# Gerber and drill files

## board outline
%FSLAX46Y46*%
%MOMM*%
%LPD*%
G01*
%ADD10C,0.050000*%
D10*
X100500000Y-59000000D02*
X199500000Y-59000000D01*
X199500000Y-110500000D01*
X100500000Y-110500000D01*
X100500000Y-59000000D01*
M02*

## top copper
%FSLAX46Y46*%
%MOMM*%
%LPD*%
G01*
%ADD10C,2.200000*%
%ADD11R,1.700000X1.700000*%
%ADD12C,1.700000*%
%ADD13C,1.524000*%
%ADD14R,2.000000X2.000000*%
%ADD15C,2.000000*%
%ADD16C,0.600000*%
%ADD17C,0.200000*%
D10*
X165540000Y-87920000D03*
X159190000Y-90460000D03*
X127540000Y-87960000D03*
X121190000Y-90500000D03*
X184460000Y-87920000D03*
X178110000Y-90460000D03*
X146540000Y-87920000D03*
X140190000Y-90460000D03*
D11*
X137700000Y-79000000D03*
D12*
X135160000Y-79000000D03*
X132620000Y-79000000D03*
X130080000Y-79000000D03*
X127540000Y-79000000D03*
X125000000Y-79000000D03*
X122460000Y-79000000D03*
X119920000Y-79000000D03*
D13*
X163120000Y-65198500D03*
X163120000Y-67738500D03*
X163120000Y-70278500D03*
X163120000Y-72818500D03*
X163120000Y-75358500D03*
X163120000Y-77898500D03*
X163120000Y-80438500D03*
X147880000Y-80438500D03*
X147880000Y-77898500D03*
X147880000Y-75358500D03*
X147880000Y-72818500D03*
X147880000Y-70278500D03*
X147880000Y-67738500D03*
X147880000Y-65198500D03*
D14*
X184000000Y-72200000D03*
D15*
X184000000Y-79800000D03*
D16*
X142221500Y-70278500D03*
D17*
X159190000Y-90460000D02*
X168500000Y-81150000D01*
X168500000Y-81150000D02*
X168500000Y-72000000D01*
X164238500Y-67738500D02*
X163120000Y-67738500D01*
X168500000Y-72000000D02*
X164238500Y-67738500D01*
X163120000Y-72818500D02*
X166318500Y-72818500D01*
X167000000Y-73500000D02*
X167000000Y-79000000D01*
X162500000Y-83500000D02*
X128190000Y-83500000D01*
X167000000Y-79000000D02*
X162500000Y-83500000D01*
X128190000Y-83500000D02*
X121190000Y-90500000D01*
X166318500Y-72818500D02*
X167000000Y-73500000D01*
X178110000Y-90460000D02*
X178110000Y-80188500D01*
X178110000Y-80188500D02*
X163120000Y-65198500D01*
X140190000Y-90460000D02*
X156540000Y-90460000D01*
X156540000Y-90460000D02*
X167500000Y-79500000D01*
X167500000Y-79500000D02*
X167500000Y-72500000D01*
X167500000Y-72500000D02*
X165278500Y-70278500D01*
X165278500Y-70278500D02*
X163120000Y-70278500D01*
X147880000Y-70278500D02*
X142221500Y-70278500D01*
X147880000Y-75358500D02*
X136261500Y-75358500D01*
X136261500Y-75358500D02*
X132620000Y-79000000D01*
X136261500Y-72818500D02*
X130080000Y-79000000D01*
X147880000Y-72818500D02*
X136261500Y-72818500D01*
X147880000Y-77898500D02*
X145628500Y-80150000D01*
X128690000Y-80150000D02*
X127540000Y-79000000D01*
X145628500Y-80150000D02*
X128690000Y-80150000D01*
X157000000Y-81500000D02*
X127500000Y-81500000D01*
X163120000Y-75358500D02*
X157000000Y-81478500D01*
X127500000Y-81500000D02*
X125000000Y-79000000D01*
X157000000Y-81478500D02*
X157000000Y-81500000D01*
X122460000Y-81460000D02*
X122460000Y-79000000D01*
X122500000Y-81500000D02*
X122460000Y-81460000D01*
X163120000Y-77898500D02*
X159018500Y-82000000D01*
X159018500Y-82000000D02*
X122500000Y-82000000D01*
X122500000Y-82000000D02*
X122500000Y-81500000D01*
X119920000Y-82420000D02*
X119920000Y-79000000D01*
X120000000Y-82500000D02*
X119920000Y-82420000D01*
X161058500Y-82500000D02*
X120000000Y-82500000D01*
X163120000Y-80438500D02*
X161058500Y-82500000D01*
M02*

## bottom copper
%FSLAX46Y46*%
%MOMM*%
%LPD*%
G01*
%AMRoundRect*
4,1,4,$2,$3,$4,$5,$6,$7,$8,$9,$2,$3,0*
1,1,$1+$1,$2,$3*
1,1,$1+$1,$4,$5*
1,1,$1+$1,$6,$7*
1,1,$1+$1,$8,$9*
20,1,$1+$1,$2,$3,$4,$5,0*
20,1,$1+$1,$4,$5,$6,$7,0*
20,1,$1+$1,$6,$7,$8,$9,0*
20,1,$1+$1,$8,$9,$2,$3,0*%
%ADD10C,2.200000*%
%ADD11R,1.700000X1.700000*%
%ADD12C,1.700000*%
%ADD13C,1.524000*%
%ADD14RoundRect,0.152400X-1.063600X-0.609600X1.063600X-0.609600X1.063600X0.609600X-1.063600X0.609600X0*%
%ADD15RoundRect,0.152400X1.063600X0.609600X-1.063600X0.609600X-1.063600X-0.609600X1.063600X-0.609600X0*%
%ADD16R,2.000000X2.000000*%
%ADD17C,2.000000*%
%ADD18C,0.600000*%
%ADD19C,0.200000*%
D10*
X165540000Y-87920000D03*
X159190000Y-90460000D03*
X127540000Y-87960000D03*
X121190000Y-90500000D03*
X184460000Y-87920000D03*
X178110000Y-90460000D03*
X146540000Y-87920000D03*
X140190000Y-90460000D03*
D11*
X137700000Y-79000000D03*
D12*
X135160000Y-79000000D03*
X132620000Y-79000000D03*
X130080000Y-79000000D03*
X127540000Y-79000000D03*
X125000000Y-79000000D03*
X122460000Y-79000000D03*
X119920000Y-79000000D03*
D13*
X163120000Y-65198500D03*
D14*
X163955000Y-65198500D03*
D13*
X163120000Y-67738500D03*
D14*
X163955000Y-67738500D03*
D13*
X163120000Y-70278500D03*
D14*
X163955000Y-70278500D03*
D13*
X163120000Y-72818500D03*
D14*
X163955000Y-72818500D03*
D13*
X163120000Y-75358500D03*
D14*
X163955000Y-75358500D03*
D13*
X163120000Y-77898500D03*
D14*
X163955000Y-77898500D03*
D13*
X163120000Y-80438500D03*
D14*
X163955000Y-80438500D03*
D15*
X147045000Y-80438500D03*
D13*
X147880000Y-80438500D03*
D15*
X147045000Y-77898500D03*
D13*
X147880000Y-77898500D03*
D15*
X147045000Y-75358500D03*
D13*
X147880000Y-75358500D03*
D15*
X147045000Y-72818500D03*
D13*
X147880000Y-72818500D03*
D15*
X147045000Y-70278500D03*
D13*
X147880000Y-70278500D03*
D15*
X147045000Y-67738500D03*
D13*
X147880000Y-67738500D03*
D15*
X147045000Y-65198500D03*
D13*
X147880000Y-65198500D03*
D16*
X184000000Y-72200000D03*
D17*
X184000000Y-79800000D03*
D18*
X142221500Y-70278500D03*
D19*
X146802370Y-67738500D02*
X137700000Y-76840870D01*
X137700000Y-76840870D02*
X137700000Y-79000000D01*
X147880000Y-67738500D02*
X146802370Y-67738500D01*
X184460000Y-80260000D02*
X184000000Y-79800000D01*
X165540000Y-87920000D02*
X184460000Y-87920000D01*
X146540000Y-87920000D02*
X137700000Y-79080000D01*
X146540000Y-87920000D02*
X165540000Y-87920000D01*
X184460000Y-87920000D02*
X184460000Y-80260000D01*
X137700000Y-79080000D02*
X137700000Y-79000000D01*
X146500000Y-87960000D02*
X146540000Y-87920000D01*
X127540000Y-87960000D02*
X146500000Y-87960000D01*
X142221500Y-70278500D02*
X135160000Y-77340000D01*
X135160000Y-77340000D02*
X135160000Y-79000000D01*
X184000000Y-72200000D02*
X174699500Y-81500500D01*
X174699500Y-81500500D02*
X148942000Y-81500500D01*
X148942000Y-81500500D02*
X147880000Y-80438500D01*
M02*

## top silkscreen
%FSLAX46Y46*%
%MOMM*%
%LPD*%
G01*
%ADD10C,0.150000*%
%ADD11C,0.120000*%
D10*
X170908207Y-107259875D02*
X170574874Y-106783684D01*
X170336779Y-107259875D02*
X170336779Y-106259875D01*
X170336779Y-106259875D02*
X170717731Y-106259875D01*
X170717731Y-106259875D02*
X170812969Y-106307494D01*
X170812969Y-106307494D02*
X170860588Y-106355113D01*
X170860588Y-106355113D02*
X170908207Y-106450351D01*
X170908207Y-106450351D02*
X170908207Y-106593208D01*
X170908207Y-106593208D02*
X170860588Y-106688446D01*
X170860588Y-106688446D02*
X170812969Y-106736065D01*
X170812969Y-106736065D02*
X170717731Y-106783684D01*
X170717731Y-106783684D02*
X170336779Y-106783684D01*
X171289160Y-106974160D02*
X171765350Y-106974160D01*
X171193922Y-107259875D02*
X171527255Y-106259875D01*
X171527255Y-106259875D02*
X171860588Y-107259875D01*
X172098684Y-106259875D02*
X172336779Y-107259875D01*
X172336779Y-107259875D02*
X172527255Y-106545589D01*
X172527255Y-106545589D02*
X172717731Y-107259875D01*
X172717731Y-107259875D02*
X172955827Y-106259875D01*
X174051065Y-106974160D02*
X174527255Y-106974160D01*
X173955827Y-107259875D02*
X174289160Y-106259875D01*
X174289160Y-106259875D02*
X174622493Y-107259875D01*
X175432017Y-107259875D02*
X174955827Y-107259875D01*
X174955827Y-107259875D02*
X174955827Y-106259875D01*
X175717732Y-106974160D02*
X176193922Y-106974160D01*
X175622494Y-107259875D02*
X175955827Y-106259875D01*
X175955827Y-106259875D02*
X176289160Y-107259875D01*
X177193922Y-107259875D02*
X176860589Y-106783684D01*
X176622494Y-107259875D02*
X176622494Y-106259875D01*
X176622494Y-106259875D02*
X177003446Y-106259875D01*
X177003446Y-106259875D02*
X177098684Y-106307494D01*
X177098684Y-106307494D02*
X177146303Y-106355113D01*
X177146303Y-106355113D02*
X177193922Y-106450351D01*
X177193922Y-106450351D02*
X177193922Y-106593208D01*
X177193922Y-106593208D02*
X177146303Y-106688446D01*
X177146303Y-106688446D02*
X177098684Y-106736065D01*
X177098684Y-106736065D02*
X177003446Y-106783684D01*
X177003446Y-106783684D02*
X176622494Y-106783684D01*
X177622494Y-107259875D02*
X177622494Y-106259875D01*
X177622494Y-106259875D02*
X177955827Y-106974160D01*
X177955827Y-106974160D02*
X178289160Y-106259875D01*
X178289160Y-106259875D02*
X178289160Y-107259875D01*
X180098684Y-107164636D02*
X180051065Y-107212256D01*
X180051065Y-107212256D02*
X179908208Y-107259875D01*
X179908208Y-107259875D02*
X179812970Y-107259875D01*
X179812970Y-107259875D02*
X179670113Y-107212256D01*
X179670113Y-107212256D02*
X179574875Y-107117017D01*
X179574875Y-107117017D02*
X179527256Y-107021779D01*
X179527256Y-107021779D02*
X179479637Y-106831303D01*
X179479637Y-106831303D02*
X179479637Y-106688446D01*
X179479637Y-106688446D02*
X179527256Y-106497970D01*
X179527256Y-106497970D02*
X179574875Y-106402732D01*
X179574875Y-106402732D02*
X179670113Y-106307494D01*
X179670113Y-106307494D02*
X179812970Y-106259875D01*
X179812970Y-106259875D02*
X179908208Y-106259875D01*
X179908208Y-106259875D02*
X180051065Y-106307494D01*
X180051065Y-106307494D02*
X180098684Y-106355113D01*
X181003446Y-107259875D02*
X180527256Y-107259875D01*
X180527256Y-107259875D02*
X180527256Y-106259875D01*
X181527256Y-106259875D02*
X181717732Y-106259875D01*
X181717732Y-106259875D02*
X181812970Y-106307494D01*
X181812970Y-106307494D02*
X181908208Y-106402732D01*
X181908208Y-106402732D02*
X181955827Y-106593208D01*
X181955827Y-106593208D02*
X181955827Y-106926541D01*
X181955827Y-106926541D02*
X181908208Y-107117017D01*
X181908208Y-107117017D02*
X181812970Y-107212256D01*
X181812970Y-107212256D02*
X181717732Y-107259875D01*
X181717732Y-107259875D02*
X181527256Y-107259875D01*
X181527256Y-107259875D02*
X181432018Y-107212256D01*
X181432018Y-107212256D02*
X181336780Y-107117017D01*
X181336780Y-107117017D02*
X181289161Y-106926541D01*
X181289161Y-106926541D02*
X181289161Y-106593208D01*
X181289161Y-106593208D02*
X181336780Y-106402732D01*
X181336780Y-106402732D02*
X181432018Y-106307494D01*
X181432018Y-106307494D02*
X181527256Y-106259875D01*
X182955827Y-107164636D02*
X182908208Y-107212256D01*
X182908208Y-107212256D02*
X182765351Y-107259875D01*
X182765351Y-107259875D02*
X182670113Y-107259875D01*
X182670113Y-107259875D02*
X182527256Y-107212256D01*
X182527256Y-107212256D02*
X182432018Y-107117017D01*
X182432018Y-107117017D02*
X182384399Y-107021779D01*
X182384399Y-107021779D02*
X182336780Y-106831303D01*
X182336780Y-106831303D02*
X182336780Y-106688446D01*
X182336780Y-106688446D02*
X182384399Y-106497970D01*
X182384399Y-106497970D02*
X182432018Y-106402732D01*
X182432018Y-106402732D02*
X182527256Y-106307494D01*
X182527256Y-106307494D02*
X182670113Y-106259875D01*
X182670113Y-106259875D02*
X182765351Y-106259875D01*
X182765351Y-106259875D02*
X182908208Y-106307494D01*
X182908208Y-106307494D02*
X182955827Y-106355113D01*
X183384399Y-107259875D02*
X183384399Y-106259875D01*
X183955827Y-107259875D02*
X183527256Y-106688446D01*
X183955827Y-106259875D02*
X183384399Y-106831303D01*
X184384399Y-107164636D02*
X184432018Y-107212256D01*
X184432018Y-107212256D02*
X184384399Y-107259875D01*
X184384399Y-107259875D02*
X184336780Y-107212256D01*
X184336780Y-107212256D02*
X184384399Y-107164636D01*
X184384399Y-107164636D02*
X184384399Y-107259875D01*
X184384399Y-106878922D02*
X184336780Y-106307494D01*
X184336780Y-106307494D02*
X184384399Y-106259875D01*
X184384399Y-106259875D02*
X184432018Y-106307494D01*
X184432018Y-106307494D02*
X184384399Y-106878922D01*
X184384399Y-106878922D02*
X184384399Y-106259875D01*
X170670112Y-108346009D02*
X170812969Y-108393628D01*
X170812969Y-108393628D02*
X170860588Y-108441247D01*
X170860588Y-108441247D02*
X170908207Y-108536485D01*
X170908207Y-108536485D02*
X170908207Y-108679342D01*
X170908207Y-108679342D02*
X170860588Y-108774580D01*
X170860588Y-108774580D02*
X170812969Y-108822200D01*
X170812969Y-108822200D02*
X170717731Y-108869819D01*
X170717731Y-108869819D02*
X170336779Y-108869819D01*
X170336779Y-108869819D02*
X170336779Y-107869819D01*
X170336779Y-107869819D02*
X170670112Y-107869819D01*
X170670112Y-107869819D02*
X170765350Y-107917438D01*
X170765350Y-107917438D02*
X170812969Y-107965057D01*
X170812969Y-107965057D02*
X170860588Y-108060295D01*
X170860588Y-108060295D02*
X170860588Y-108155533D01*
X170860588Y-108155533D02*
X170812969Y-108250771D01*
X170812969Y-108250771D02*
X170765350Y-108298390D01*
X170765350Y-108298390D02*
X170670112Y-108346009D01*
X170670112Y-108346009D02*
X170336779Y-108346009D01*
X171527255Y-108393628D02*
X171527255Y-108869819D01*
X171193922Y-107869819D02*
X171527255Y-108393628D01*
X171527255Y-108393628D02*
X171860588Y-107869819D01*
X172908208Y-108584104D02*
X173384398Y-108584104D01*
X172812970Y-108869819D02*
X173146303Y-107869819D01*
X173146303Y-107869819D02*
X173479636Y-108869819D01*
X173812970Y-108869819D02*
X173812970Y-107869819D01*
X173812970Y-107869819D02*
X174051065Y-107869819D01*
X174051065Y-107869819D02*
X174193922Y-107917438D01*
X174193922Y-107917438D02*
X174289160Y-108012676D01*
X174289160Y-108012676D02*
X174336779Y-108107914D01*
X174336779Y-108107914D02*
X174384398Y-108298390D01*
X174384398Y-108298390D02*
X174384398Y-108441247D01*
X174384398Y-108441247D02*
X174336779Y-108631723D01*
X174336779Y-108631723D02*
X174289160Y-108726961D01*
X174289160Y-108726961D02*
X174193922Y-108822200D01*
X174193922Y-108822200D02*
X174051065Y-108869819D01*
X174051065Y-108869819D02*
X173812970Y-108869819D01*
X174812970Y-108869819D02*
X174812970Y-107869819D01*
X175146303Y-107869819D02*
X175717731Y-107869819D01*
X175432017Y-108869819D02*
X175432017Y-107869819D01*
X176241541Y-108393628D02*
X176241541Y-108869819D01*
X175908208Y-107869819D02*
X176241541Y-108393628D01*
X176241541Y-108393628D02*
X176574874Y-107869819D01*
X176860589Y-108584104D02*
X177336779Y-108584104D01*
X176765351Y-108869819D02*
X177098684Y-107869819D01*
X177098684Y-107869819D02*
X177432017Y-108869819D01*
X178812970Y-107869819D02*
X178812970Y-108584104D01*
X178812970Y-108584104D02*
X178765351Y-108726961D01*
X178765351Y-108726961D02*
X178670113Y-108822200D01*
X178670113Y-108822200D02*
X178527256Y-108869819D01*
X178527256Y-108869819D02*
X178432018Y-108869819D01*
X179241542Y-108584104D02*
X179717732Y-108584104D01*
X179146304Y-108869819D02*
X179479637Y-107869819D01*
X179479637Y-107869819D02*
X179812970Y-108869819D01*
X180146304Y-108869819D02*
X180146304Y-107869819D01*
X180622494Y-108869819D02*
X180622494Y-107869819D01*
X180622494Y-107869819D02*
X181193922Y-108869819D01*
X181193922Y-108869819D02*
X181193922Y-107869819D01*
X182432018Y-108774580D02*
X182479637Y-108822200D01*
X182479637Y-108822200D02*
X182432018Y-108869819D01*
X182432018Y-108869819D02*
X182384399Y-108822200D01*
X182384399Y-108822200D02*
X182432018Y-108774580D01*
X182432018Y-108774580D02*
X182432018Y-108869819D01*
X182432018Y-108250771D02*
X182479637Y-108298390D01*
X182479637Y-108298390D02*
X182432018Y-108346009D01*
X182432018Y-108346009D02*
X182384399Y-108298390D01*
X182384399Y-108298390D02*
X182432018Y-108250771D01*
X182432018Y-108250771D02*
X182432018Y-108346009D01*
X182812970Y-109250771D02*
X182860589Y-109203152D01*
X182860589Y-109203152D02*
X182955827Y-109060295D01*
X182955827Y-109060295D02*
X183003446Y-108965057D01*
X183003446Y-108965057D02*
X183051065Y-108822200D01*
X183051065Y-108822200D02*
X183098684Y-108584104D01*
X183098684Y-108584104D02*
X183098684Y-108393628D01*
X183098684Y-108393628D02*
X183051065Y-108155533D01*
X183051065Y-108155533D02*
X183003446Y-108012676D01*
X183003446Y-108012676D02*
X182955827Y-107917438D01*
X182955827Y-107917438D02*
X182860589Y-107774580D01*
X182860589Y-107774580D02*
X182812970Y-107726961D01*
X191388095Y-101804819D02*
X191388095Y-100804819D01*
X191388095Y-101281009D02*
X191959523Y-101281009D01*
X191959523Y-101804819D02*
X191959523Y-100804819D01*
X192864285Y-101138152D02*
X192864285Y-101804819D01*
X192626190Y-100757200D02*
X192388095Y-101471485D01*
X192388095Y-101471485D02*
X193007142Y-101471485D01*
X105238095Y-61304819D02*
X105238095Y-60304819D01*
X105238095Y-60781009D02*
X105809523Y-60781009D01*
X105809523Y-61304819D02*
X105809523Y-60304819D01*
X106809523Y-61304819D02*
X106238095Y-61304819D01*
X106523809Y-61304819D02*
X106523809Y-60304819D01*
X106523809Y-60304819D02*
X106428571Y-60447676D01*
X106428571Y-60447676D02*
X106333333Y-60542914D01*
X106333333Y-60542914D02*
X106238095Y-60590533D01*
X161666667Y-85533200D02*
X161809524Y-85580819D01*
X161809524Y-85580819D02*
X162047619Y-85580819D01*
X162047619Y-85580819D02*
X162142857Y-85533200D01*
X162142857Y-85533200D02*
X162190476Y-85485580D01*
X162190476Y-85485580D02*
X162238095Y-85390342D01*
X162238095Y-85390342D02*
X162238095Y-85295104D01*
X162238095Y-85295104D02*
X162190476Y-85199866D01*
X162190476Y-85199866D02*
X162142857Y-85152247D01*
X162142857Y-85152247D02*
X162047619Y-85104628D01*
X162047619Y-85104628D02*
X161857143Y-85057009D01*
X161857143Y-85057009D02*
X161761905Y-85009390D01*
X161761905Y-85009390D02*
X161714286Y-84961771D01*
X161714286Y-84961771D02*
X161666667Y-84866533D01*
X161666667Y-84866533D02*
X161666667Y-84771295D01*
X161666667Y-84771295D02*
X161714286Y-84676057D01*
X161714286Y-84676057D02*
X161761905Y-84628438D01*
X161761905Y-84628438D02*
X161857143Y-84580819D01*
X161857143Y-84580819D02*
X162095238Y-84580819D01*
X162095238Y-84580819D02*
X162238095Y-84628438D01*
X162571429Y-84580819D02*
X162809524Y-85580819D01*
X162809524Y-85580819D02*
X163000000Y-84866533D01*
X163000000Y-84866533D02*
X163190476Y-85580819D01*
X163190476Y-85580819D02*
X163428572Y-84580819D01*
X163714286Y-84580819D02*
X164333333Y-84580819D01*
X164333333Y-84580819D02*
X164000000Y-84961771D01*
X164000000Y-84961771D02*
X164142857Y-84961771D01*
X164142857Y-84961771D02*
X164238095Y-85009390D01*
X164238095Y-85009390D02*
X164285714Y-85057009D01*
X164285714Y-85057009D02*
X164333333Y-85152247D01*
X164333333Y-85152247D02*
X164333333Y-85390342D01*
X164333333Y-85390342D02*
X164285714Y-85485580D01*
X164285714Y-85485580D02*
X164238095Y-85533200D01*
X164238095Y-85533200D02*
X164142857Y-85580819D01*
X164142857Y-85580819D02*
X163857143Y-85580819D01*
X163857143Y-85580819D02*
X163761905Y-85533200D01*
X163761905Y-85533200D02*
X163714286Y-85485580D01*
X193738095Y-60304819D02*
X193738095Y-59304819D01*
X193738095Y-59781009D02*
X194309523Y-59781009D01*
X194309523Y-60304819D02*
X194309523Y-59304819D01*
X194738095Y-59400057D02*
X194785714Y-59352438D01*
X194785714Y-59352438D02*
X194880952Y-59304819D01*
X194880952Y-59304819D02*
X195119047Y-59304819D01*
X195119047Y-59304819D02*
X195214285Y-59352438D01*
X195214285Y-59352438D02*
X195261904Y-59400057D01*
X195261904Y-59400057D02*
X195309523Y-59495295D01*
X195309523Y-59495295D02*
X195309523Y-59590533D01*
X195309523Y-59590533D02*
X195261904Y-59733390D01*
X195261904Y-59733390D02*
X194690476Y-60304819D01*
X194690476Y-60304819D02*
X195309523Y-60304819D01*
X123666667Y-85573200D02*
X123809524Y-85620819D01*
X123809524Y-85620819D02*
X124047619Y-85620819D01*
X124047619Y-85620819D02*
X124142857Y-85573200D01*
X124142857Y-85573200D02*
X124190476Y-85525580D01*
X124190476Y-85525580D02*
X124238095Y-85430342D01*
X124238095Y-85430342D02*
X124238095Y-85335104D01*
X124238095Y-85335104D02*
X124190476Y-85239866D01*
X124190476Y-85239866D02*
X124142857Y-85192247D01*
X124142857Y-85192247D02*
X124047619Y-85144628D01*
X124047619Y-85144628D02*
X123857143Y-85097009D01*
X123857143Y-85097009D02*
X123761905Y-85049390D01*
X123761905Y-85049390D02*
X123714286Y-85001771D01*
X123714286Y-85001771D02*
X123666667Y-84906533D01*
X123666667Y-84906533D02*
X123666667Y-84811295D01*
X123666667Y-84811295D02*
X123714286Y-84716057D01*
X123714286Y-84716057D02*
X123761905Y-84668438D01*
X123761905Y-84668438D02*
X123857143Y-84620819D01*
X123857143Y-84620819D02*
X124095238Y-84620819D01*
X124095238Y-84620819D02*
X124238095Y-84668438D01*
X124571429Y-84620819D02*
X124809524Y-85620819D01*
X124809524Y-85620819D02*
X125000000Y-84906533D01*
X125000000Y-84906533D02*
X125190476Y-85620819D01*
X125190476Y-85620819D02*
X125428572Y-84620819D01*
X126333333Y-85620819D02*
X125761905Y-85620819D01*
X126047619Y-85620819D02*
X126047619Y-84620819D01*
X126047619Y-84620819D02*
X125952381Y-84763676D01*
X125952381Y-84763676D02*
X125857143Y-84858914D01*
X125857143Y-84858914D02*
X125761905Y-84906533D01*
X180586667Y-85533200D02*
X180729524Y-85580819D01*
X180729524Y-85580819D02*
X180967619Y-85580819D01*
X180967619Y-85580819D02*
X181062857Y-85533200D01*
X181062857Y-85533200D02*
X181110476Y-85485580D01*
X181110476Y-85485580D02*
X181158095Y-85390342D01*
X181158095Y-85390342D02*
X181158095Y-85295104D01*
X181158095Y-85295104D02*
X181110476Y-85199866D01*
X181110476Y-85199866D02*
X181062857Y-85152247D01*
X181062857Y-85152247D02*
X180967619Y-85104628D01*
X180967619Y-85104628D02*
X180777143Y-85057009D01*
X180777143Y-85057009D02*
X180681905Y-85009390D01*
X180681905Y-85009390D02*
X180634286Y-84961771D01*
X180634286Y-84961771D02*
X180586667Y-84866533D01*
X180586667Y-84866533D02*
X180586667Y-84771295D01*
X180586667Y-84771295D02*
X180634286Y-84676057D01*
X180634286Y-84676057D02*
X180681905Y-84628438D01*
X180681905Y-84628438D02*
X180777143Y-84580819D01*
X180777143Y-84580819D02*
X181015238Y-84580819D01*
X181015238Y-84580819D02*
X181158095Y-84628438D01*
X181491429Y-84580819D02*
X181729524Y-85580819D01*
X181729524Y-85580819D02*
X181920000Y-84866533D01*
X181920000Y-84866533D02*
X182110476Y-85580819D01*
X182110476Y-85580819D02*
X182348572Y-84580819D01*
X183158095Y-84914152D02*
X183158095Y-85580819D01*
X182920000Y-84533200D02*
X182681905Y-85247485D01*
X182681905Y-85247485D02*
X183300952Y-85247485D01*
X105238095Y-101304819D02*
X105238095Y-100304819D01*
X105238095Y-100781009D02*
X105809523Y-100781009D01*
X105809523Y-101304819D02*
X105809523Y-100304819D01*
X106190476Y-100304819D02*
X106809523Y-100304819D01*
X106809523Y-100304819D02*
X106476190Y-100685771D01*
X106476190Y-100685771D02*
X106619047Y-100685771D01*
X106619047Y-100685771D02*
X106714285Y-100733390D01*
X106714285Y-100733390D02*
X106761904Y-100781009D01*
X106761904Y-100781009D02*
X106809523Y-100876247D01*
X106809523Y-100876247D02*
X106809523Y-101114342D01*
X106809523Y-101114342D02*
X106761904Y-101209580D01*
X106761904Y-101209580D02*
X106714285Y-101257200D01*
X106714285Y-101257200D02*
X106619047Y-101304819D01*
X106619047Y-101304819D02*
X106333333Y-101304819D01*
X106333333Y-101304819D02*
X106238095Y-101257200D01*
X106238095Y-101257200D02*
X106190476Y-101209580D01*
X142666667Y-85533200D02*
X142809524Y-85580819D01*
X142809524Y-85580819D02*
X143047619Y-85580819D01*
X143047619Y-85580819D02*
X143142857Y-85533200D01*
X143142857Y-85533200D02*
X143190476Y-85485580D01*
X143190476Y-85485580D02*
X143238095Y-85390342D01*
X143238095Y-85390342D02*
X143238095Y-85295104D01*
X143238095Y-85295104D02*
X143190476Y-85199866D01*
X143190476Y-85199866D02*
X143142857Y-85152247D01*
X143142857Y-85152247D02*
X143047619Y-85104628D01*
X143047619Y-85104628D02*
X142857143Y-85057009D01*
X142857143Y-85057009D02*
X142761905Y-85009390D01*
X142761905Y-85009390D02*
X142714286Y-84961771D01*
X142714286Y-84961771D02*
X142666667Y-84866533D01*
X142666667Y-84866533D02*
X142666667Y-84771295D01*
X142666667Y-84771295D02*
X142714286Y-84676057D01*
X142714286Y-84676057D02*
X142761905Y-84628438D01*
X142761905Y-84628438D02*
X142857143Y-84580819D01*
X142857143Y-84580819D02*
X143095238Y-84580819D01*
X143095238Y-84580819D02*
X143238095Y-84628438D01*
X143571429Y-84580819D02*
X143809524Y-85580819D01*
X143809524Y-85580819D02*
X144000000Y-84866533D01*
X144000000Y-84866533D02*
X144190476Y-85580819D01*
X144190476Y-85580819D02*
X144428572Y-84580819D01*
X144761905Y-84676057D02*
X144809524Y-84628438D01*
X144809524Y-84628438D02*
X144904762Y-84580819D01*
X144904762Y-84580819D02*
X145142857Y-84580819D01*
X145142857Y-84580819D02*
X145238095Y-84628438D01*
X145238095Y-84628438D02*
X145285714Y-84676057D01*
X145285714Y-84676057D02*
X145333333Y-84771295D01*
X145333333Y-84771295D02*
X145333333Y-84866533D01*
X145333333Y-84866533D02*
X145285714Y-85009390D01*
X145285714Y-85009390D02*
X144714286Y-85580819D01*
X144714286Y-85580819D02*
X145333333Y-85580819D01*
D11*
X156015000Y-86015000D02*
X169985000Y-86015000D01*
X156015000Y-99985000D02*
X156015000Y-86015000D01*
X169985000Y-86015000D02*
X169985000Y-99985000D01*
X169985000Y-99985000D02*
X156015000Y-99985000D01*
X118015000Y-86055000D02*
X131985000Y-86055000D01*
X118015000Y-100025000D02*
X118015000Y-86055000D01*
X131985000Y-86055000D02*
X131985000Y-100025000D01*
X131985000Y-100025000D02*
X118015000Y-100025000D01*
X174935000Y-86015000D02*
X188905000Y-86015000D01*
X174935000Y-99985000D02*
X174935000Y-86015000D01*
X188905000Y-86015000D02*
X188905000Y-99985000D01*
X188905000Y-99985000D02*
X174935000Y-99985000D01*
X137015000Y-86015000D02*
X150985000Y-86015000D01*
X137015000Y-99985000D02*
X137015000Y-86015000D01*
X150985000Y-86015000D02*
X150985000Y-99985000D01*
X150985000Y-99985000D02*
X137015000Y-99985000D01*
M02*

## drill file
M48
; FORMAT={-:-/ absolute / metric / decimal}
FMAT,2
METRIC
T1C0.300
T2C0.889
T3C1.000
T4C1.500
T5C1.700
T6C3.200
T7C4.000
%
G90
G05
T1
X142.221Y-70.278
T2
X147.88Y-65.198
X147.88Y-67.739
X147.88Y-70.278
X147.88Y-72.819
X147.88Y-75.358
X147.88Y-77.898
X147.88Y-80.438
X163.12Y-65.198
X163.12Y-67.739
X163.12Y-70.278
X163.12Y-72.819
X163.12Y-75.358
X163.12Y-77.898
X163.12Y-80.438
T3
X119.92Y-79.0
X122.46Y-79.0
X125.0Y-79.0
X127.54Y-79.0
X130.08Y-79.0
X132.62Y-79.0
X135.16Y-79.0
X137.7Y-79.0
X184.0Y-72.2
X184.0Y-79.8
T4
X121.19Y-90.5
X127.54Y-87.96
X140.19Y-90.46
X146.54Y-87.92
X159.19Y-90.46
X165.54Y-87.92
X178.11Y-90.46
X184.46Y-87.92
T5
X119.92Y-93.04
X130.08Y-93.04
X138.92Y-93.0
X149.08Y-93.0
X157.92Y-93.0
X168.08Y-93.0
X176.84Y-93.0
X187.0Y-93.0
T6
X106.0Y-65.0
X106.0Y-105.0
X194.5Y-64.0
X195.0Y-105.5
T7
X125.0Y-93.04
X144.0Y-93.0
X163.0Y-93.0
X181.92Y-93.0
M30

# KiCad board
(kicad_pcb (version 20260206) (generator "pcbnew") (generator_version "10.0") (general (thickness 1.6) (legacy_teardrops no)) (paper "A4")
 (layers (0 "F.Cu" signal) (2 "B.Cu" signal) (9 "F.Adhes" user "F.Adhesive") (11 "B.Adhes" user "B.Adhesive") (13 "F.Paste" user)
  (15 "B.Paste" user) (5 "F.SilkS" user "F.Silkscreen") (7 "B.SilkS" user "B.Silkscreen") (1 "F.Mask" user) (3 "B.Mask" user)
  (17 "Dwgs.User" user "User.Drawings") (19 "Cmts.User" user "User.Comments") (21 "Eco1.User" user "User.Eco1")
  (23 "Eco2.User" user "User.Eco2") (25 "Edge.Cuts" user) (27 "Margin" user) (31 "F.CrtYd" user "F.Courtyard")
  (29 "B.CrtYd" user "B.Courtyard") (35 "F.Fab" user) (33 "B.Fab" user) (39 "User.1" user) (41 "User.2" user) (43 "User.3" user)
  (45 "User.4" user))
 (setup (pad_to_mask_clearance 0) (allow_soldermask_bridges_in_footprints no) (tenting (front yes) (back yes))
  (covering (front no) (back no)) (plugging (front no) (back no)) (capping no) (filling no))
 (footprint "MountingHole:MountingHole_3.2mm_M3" (layer "F.Cu") (at 195 105.5)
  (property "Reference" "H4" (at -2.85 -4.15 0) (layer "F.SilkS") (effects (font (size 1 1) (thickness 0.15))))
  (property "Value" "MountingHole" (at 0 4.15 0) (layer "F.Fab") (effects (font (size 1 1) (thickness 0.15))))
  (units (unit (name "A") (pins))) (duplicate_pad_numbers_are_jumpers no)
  (pad "" np_thru_hole circle (at 0 0) (size 3.2 3.2) (drill 3.2) (layers "*.Cu" "*.Mask")))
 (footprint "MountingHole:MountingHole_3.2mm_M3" (layer "F.Cu") (at 106 65)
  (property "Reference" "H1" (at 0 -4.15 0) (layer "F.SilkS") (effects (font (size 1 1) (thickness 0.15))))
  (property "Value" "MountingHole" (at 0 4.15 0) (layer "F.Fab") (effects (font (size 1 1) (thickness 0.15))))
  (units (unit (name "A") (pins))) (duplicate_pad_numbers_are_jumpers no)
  (pad "" np_thru_hole circle (at 0 0) (size 3.2 3.2) (drill 3.2) (layers "*.Cu" "*.Mask")))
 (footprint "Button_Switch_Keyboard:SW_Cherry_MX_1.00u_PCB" (layer "F.Cu") (at 165.54 87.92)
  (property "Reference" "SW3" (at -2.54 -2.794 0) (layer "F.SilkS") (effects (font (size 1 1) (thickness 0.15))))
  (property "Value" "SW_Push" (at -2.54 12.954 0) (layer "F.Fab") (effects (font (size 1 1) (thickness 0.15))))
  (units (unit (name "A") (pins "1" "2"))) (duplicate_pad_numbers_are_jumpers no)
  (fp_line (start -9.525 -1.905) (end 4.445 -1.905) (stroke (width 0.12) (type solid)) (layer "F.SilkS"))
  (fp_line (start -9.525 12.065) (end -9.525 -1.905) (stroke (width 0.12) (type solid)) (layer "F.SilkS"))
  (fp_line (start 4.445 -1.905) (end 4.445 12.065) (stroke (width 0.12) (type solid)) (layer "F.SilkS"))
  (fp_line (start 4.445 12.065) (end -9.525 12.065) (stroke (width 0.12) (type solid)) (layer "F.SilkS"))
  (pad "" np_thru_hole circle (at -7.62 5.08) (size 1.7 1.7) (drill 1.7) (layers "*.Cu" "*.Mask"))
  (pad "" np_thru_hole circle (at -2.54 5.08) (size 4 4) (drill 4) (layers "*.Cu" "*.Mask"))
  (pad "" np_thru_hole circle (at 2.54 5.08) (size 1.7 1.7) (drill 1.7) (layers "*.Cu" "*.Mask"))
  (pad "1" thru_hole circle (at 0 0) (size 2.2 2.2) (drill 1.5) (layers "*.Cu" "*.Mask") (remove_unused_layers no) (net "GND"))
  (pad "2" thru_hole circle (at -6.35 2.54) (size 2.2 2.2) (drill 1.5) (layers "*.Cu" "*.Mask") (remove_unused_layers no)
   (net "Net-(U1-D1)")))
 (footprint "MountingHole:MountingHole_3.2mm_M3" (layer "F.Cu") (at 194.5 64)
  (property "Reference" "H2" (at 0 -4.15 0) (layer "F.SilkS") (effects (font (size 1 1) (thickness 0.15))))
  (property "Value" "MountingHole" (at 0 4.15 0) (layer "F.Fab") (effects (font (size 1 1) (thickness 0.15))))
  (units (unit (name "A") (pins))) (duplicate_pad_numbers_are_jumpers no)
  (pad "" np_thru_hole circle (at 0 0) (size 3.2 3.2) (drill 3.2) (layers "*.Cu" "*.Mask")))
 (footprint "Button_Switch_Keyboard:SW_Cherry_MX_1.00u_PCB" (layer "F.Cu") (at 127.54 87.96)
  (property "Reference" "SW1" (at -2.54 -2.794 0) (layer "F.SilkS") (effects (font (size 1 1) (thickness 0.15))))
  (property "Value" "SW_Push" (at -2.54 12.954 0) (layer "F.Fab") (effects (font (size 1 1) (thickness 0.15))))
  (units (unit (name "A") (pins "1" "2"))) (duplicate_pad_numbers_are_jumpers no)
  (fp_line (start -9.525 -1.905) (end 4.445 -1.905) (stroke (width 0.12) (type solid)) (layer "F.SilkS"))
  (fp_line (start -9.525 12.065) (end -9.525 -1.905) (stroke (width 0.12) (type solid)) (layer "F.SilkS"))
  (fp_line (start 4.445 -1.905) (end 4.445 12.065) (stroke (width 0.12) (type solid)) (layer "F.SilkS"))
  (fp_line (start 4.445 12.065) (end -9.525 12.065) (stroke (width 0.12) (type solid)) (layer "F.SilkS"))
  (pad "" np_thru_hole circle (at -7.62 5.08) (size 1.7 1.7) (drill 1.7) (layers "*.Cu" "*.Mask"))
  (pad "" np_thru_hole circle (at -2.54 5.08) (size 4 4) (drill 4) (layers "*.Cu" "*.Mask"))
  (pad "" np_thru_hole circle (at 2.54 5.08) (size 1.7 1.7) (drill 1.7) (layers "*.Cu" "*.Mask"))
  (pad "1" thru_hole circle (at 0 0) (size 2.2 2.2) (drill 1.5) (layers "*.Cu" "*.Mask") (remove_unused_layers no) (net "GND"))
  (pad "2" thru_hole circle (at -6.35 2.54) (size 2.2 2.2) (drill 1.5) (layers "*.Cu" "*.Mask") (remove_unused_layers no)
   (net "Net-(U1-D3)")))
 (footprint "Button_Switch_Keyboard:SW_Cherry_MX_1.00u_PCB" (layer "F.Cu") (at 184.46 87.92)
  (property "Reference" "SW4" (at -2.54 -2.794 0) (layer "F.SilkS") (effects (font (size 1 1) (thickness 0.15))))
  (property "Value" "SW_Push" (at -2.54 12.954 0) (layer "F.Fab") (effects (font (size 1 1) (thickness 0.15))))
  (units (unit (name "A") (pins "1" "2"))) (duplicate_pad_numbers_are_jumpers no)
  (fp_line (start -9.525 -1.905) (end 4.445 -1.905) (stroke (width 0.12) (type solid)) (layer "F.SilkS"))
  (fp_line (start -9.525 12.065) (end -9.525 -1.905) (stroke (width 0.12) (type solid)) (layer "F.SilkS"))
  (fp_line (start 4.445 -1.905) (end 4.445 12.065) (stroke (width 0.12) (type solid)) (layer "F.SilkS"))
  (fp_line (start 4.445 12.065) (end -9.525 12.065) (stroke (width 0.12) (type solid)) (layer "F.SilkS"))
  (pad "" np_thru_hole circle (at -7.62 5.08) (size 1.7 1.7) (drill 1.7) (layers "*.Cu" "*.Mask"))
  (pad "" np_thru_hole circle (at -2.54 5.08) (size 4 4) (drill 4) (layers "*.Cu" "*.Mask"))
  (pad "" np_thru_hole circle (at 2.54 5.08) (size 1.7 1.7) (drill 1.7) (layers "*.Cu" "*.Mask"))
  (pad "1" thru_hole circle (at 0 0) (size 2.2 2.2) (drill 1.5) (layers "*.Cu" "*.Mask") (remove_unused_layers no) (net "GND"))
  (pad "2" thru_hole circle (at -6.35 2.54) (size 2.2 2.2) (drill 1.5) (layers "*.Cu" "*.Mask") (remove_unused_layers no)
   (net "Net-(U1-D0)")))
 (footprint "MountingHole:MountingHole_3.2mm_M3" (layer "F.Cu") (at 106 105)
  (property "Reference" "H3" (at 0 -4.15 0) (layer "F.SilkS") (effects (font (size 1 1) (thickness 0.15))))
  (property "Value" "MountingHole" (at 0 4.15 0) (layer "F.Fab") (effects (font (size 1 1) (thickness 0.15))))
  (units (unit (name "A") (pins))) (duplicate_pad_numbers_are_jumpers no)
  (pad "" np_thru_hole circle (at 0 0) (size 3.2 3.2) (drill 3.2) (layers "*.Cu" "*.Mask")))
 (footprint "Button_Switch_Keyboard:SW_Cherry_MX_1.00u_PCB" (layer "F.Cu") (at 146.54 87.92)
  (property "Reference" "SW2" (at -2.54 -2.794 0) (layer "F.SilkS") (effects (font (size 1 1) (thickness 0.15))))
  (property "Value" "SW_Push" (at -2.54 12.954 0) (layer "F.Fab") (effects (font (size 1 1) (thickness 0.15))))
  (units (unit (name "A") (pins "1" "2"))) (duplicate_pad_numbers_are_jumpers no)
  (fp_line (start -9.525 -1.905) (end 4.445 -1.905) (stroke (width 0.12) (type solid)) (layer "F.SilkS"))
  (fp_line (start -9.525 12.065) (end -9.525 -1.905) (stroke (width 0.12) (type solid)) (layer "F.SilkS"))
  (fp_line (start 4.445 -1.905) (end 4.445 12.065) (stroke (width 0.12) (type solid)) (layer "F.SilkS"))
  (fp_line (start 4.445 12.065) (end -9.525 12.065) (stroke (width 0.12) (type solid)) (layer "F.SilkS"))
  (pad "" np_thru_hole circle (at -7.62 5.08) (size 1.7 1.7) (drill 1.7) (layers "*.Cu" "*.Mask"))
  (pad "" np_thru_hole circle (at -2.54 5.08) (size 4 4) (drill 4) (layers "*.Cu" "*.Mask"))
  (pad "" np_thru_hole circle (at 2.54 5.08) (size 1.7 1.7) (drill 1.7) (layers "*.Cu" "*.Mask"))
  (pad "1" thru_hole circle (at 0 0) (size 2.2 2.2) (drill 1.5) (layers "*.Cu" "*.Mask") (remove_unused_layers no) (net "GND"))
  (pad "2" thru_hole circle (at -6.35 2.54) (size 2.2 2.2) (drill 1.5) (layers "*.Cu" "*.Mask") (remove_unused_layers no)
   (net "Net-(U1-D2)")))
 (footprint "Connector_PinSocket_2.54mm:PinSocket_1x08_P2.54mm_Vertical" (layer "B.Cu") (at 137.7 79 90)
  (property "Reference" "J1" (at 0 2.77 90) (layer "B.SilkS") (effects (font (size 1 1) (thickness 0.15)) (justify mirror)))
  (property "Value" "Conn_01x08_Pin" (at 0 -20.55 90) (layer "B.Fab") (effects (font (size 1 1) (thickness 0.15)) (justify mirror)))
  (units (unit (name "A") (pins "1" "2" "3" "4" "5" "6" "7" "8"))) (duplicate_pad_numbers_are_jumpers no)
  (pad "1" thru_hole rect (at 0 0 90) (size 1.7 1.7) (drill 1) (layers "*.Cu" "*.Mask") (remove_unused_layers no) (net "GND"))
  (pad "2" thru_hole circle (at 0 -2.54 90) (size 1.7 1.7) (drill 1) (layers "*.Cu" "*.Mask") (remove_unused_layers no) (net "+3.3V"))
  (pad "3" thru_hole circle (at 0 -5.08 90) (size 1.7 1.7) (drill 1) (layers "*.Cu" "*.Mask") (remove_unused_layers no) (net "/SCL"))
  (pad "4" thru_hole circle (at 0 -7.62 90) (size 1.7 1.7) (drill 1) (layers "*.Cu" "*.Mask") (remove_unused_layers no) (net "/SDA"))
  (pad "5" thru_hole circle (at 0 -10.16 90) (size 1.7 1.7) (drill 1) (layers "*.Cu" "*.Mask") (remove_unused_layers no) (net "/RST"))
  (pad "6" thru_hole circle (at 0 -12.7 90) (size 1.7 1.7) (drill 1) (layers "*.Cu" "*.Mask") (remove_unused_layers no) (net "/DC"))
  (pad "7" thru_hole circle (at 0 -15.24 90) (size 1.7 1.7) (drill 1) (layers "*.Cu" "*.Mask") (remove_unused_layers no) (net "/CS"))
  (pad "8" thru_hole circle (at 0 -17.78 90) (size 1.7 1.7) (drill 1) (layers "*.Cu" "*.Mask") (remove_unused_layers no) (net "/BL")))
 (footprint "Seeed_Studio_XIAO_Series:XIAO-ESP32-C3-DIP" (layer "B.Cu") (at 155.5 72.8185 90)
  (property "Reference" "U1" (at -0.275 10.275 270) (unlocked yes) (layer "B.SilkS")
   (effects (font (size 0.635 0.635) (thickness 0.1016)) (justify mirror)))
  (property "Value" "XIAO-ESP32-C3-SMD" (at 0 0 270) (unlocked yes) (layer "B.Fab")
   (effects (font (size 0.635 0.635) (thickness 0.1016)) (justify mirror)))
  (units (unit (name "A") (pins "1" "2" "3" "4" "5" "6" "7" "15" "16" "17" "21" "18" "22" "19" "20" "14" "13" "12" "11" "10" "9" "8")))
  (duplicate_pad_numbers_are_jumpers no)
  (pad "1" thru_hole circle (at 7.62 7.62) (size 1.524 1.524) (drill 0.889) (layers "*.Cu" "*.Mask") (remove_unused_layers no)
   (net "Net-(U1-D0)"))
  (pad "1" smd roundrect (at 7.62 8.455) (size 2.432 1.524) (layers "B.Cu" "B.Mask") (roundrect_rratio 0.1) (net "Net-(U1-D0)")
   (thermal_bridge_angle 45))
  (pad "2" thru_hole circle (at 5.08 7.62) (size 1.524 1.524) (drill 0.889) (layers "*.Cu" "*.Mask") (remove_unused_layers no)
   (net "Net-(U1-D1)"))
  (pad "2" smd roundrect (at 5.08 8.455) (size 2.432 1.524) (layers "B.Cu" "B.Mask") (roundrect_rratio 0.1) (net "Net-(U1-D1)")
   (thermal_bridge_angle 45))
  (pad "3" thru_hole circle (at 2.54 7.62) (size 1.524 1.524) (drill 0.889) (layers "*.Cu" "*.Mask") (remove_unused_layers no)
   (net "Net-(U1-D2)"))
  (pad "3" smd roundrect (at 2.54 8.455) (size 2.432 1.524) (layers "B.Cu" "B.Mask") (roundrect_rratio 0.1) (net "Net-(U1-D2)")
   (thermal_bridge_angle 45))
  (pad "4" thru_hole circle (at 0 7.62) (size 1.524 1.524) (drill 0.889) (layers "*.Cu" "*.Mask") (remove_unused_layers no)
   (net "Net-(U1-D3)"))
  (pad "4" smd roundrect (at 0 8.455) (size 2.432 1.524) (layers "B.Cu" "B.Mask") (roundrect_rratio 0.1) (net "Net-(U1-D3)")
   (thermal_bridge_angle 45))
  (pad "5" thru_hole circle (at -2.54 7.62) (size 1.524 1.524) (drill 0.889) (layers "*.Cu" "*.Mask") (remove_unused_layers no) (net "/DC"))
  (pad "5" smd roundrect (at -2.54 8.455) (size 2.432 1.524) (layers "B.Cu" "B.Mask") (roundrect_rratio 0.1) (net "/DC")
   (thermal_bridge_angle 45))
  (pad "6" thru_hole circle (at -5.08 7.62) (size 1.524 1.524) (drill 0.889) (layers "*.Cu" "*.Mask") (remove_unused_layers no) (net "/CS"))
  (pad "6" smd roundrect (at -5.08 8.455) (size 2.432 1.524) (layers "B.Cu" "B.Mask") (roundrect_rratio 0.1) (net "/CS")
   (thermal_bridge_angle 45))
  (pad "7" thru_hole circle (at -7.62 7.62) (size 1.524 1.524) (drill 0.889) (layers "*.Cu" "*.Mask") (remove_unused_layers no) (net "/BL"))
  (pad "7" smd roundrect (at -7.62 8.455) (size 2.432 1.524) (layers "B.Cu" "B.Mask") (roundrect_rratio 0.1) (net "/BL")
   (thermal_bridge_angle 45))
  (pad "8" smd roundrect (at -7.62 -8.455 180) (size 2.432 1.524) (layers "B.Cu" "B.Mask") (roundrect_rratio 0.1) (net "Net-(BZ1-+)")
   (thermal_bridge_angle 45))
  (pad "8" thru_hole circle (at -7.62 -7.62 180) (size 1.524 1.524) (drill 0.889) (layers "*.Cu" "*.Mask") (remove_unused_layers no)
   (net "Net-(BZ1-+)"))
  (pad "9" smd roundrect (at -5.08 -8.455 180) (size 2.432 1.524) (layers "B.Cu" "B.Mask") (roundrect_rratio 0.1) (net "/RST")
   (thermal_bridge_angle 45))
  (pad "9" thru_hole circle (at -5.08 -7.62 180) (size 1.524 1.524) (drill 0.889) (layers "*.Cu" "*.Mask") (remove_unused_layers no)
   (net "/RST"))
  (pad "10" smd roundrect (at -2.54 -8.455 180) (size 2.432 1.524) (layers "B.Cu" "B.Mask") (roundrect_rratio 0.1) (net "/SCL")
   (thermal_bridge_angle 45))
  (pad "10" thru_hole circle (at -2.54 -7.62 180) (size 1.524 1.524) (drill 0.889) (layers "*.Cu" "*.Mask") (remove_unused_layers no)
   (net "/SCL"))
  (pad "11" smd roundrect (at 0 -8.455 180) (size 2.432 1.524) (layers "B.Cu" "B.Mask") (roundrect_rratio 0.1) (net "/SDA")
   (thermal_bridge_angle 45))
  (pad "11" thru_hole circle (at 0 -7.62 180) (size 1.524 1.524) (drill 0.889) (layers "*.Cu" "*.Mask") (remove_unused_layers no)
   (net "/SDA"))
  (pad "12" smd roundrect (at 2.54 -8.455 180) (size 2.432 1.524) (layers "B.Cu" "B.Mask") (roundrect_rratio 0.1) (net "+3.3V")
   (thermal_bridge_angle 45))
  (pad "12" thru_hole circle (at 2.54 -7.62 180) (size 1.524 1.524) (drill 0.889) (layers "*.Cu" "*.Mask") (remove_unused_layers no)
   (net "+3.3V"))
  (pad "13" smd roundrect (at 5.08 -8.455 180) (size 2.432 1.524) (layers "B.Cu" "B.Mask") (roundrect_rratio 0.1) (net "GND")
   (thermal_bridge_angle 45))
  (pad "13" thru_hole circle (at 5.08 -7.62 180) (size 1.524 1.524) (drill 0.889) (layers "*.Cu" "*.Mask") (remove_unused_layers no)
   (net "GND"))
  (pad "14" smd roundrect (at 7.62 -8.455 180) (size 2.432 1.524) (layers "B.Cu" "B.Mask") (roundrect_rratio 0.1)
   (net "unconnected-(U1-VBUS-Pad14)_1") (thermal_bridge_angle 45))
  (pad "14" thru_hole circle (at 7.62 -7.62 180) (size 1.524 1.524) (drill 0.889) (layers "*.Cu" "*.Mask") (remove_unused_layers no)
   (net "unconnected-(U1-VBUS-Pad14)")))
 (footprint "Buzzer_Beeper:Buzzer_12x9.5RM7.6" (layer "B.Cu") (at 184 72.2 -90)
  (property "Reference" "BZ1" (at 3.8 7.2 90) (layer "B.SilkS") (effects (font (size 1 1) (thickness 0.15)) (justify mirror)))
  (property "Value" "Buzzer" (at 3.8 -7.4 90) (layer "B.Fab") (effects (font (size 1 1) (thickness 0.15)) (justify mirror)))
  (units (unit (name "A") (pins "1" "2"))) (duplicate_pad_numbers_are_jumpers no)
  (pad "1" thru_hole rect (at 0 0 270) (size 2 2) (drill 1) (layers "*.Cu" "*.Mask") (remove_unused_layers no) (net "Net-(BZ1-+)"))
  (pad "2" thru_hole circle (at 7.6 0 270) (size 2 2) (drill 1) (layers "*.Cu" "*.Mask") (remove_unused_layers no) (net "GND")))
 (gr_rect (start 100.5 59) (end 199.5 110.5) (stroke (width 0.05) (type default)) (fill no) (layer "Edge.Cuts"))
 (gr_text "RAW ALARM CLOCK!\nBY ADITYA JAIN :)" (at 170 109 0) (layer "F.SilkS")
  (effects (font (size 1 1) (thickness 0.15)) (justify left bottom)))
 (segment (start 146.80237 67.7385) (end 137.7 76.84087) (width 0.2) (layer "B.Cu") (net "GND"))
 (segment (start 137.7 76.84087) (end 137.7 79) (width 0.2) (layer "B.Cu") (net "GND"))
 (segment (start 147.88 67.7385) (end 146.80237 67.7385) (width 0.2) (layer "B.Cu") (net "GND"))
 (segment (start 184.46 80.26) (end 184 79.8) (width 0.2) (layer "B.Cu") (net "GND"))
 (segment (start 165.54 87.92) (end 184.46 87.92) (width 0.2) (layer "B.Cu") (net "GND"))
 (segment (start 146.54 87.92) (end 137.7 79.08) (width 0.2) (layer "B.Cu") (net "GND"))
 (segment (start 146.54 87.92) (end 165.54 87.92) (width 0.2) (layer "B.Cu") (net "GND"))
 (segment (start 184.46 87.92) (end 184.46 80.26) (width 0.2) (layer "B.Cu") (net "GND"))
 (segment (start 137.7 79.08) (end 137.7 79) (width 0.2) (layer "B.Cu") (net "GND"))
 (segment (start 146.5 87.96) (end 146.54 87.92) (width 0.2) (layer "B.Cu") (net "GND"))
 (segment (start 127.54 87.96) (end 146.5 87.96) (width 0.2) (layer "B.Cu") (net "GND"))
 (segment (start 159.19 90.46) (end 168.5 81.15) (width 0.2) (layer "F.Cu") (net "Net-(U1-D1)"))
 (segment (start 168.5 81.15) (end 168.5 72) (width 0.2) (layer "F.Cu") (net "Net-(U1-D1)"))
 (segment (start 164.2385 67.7385) (end 163.12 67.7385) (width 0.2) (layer "F.Cu") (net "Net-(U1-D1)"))
 (segment (start 168.5 72) (end 164.2385 67.7385) (width 0.2) (layer "F.Cu") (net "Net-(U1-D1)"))
 (segment (start 163.12 72.8185) (end 166.3185 72.8185) (width 0.2) (layer "F.Cu") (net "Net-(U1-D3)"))
 (segment (start 167 73.5) (end 167 79) (width 0.2) (layer "F.Cu") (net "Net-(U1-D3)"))
 (segment (start 162.5 83.5) (end 128.19 83.5) (width 0.2) (layer "F.Cu") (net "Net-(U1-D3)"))
 (segment (start 167 79) (end 162.5 83.5) (width 0.2) (layer "F.Cu") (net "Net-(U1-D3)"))
 (segment (start 128.19 83.5) (end 121.19 90.5) (width 0.2) (layer "F.Cu") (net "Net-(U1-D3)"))
 (segment (start 166.3185 72.8185) (end 167 73.5) (width 0.2) (layer "F.Cu") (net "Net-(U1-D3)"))
 (segment (start 178.11 90.46) (end 178.11 80.1885) (width 0.2) (layer "F.Cu") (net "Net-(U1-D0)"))
 (segment (start 178.11 80.1885) (end 163.12 65.1985) (width 0.2) (layer "F.Cu") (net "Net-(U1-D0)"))
 (segment (start 140.19 90.46) (end 156.54 90.46) (width 0.2) (layer "F.Cu") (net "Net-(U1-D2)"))
 (segment (start 156.54 90.46) (end 167.5 79.5) (width 0.2) (layer "F.Cu") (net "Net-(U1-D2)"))
 (segment (start 167.5 79.5) (end 167.5 72.5) (width 0.2) (layer "F.Cu") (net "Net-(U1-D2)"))
 (segment (start 167.5 72.5) (end 165.2785 70.2785) (width 0.2) (layer "F.Cu") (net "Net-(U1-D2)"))
 (segment (start 165.2785 70.2785) (end 163.12 70.2785) (width 0.2) (layer "F.Cu") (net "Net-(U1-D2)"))
 (segment (start 147.88 70.2785) (end 142.2215 70.2785) (width 0.2) (layer "F.Cu") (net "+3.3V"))
 (via (at 142.2215 70.2785) (size 0.6) (drill 0.3) (layers "F.Cu" "B.Cu") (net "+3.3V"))
 (segment (start 142.2215 70.2785) (end 135.16 77.34) (width 0.2) (layer "B.Cu") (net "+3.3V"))
 (segment (start 135.16 77.34) (end 135.16 79) (width 0.2) (layer "B.Cu") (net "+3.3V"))
 (segment (start 147.88 75.3585) (end 136.2615 75.3585) (width 0.2) (layer "F.Cu") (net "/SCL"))
 (segment (start 136.2615 75.3585) (end 132.62 79) (width 0.2) (layer "F.Cu") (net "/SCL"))
 (segment (start 136.2615 72.8185) (end 130.08 79) (width 0.2) (layer "F.Cu") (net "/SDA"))
 (segment (start 147.88 72.8185) (end 136.2615 72.8185) (width 0.2) (layer "F.Cu") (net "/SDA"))
 (segment (start 147.88 77.8985) (end 145.6285 80.15) (width 0.2) (layer "F.Cu") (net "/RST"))
 (segment (start 128.69 80.15) (end 127.54 79) (width 0.2) (layer "F.Cu") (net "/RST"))
 (segment (start 145.6285 80.15) (end 128.69 80.15) (width 0.2) (layer "F.Cu") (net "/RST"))
 (segment (start 157 81.5) (end 127.5 81.5) (width 0.2) (layer "F.Cu") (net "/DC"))
 (segment (start 163.12 75.3585) (end 157 81.4785) (width 0.2) (layer "F.Cu") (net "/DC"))
 (segment (start 127.5 81.5) (end 125 79) (width 0.2) (layer "F.Cu") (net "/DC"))
 (segment (start 157 81.4785) (end 157 81.5) (width 0.2) (layer "F.Cu") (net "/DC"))
 (segment (start 122.46 81.46) (end 122.46 79) (width 0.2) (layer "F.Cu") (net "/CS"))
 (segment (start 122.5 81.5) (end 122.46 81.46) (width 0.2) (layer "F.Cu") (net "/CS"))
 (segment (start 163.12 77.8985) (end 159.0185 82) (width 0.2) (layer "F.Cu") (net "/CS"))
 (segment (start 159.0185 82) (end 122.5 82) (width 0.2) (layer "F.Cu") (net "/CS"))
 (segment (start 122.5 82) (end 122.5 81.5) (width 0.2) (layer "F.Cu") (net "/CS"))
 (segment (start 119.92 82.42) (end 119.92 79) (width 0.2) (layer "F.Cu") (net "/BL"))
 (segment (start 120 82.5) (end 119.92 82.42) (width 0.2) (layer "F.Cu") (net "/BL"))
 (segment (start 161.0585 82.5) (end 120 82.5) (width 0.2) (layer "F.Cu") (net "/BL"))
 (segment (start 163.12 80.4385) (end 161.0585 82.5) (width 0.2) (layer "F.Cu") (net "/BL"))
 (segment (start 184 72.2) (end 174.6995 81.5005) (width 0.2) (layer "B.Cu") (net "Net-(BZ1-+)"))
 (segment (start 174.6995 81.5005) (end 148.942 81.5005) (width 0.2) (layer "B.Cu") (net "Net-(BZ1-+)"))
 (segment (start 148.942 81.5005) (end 147.88 80.4385) (width 0.2) (layer "B.Cu") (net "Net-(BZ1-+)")))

